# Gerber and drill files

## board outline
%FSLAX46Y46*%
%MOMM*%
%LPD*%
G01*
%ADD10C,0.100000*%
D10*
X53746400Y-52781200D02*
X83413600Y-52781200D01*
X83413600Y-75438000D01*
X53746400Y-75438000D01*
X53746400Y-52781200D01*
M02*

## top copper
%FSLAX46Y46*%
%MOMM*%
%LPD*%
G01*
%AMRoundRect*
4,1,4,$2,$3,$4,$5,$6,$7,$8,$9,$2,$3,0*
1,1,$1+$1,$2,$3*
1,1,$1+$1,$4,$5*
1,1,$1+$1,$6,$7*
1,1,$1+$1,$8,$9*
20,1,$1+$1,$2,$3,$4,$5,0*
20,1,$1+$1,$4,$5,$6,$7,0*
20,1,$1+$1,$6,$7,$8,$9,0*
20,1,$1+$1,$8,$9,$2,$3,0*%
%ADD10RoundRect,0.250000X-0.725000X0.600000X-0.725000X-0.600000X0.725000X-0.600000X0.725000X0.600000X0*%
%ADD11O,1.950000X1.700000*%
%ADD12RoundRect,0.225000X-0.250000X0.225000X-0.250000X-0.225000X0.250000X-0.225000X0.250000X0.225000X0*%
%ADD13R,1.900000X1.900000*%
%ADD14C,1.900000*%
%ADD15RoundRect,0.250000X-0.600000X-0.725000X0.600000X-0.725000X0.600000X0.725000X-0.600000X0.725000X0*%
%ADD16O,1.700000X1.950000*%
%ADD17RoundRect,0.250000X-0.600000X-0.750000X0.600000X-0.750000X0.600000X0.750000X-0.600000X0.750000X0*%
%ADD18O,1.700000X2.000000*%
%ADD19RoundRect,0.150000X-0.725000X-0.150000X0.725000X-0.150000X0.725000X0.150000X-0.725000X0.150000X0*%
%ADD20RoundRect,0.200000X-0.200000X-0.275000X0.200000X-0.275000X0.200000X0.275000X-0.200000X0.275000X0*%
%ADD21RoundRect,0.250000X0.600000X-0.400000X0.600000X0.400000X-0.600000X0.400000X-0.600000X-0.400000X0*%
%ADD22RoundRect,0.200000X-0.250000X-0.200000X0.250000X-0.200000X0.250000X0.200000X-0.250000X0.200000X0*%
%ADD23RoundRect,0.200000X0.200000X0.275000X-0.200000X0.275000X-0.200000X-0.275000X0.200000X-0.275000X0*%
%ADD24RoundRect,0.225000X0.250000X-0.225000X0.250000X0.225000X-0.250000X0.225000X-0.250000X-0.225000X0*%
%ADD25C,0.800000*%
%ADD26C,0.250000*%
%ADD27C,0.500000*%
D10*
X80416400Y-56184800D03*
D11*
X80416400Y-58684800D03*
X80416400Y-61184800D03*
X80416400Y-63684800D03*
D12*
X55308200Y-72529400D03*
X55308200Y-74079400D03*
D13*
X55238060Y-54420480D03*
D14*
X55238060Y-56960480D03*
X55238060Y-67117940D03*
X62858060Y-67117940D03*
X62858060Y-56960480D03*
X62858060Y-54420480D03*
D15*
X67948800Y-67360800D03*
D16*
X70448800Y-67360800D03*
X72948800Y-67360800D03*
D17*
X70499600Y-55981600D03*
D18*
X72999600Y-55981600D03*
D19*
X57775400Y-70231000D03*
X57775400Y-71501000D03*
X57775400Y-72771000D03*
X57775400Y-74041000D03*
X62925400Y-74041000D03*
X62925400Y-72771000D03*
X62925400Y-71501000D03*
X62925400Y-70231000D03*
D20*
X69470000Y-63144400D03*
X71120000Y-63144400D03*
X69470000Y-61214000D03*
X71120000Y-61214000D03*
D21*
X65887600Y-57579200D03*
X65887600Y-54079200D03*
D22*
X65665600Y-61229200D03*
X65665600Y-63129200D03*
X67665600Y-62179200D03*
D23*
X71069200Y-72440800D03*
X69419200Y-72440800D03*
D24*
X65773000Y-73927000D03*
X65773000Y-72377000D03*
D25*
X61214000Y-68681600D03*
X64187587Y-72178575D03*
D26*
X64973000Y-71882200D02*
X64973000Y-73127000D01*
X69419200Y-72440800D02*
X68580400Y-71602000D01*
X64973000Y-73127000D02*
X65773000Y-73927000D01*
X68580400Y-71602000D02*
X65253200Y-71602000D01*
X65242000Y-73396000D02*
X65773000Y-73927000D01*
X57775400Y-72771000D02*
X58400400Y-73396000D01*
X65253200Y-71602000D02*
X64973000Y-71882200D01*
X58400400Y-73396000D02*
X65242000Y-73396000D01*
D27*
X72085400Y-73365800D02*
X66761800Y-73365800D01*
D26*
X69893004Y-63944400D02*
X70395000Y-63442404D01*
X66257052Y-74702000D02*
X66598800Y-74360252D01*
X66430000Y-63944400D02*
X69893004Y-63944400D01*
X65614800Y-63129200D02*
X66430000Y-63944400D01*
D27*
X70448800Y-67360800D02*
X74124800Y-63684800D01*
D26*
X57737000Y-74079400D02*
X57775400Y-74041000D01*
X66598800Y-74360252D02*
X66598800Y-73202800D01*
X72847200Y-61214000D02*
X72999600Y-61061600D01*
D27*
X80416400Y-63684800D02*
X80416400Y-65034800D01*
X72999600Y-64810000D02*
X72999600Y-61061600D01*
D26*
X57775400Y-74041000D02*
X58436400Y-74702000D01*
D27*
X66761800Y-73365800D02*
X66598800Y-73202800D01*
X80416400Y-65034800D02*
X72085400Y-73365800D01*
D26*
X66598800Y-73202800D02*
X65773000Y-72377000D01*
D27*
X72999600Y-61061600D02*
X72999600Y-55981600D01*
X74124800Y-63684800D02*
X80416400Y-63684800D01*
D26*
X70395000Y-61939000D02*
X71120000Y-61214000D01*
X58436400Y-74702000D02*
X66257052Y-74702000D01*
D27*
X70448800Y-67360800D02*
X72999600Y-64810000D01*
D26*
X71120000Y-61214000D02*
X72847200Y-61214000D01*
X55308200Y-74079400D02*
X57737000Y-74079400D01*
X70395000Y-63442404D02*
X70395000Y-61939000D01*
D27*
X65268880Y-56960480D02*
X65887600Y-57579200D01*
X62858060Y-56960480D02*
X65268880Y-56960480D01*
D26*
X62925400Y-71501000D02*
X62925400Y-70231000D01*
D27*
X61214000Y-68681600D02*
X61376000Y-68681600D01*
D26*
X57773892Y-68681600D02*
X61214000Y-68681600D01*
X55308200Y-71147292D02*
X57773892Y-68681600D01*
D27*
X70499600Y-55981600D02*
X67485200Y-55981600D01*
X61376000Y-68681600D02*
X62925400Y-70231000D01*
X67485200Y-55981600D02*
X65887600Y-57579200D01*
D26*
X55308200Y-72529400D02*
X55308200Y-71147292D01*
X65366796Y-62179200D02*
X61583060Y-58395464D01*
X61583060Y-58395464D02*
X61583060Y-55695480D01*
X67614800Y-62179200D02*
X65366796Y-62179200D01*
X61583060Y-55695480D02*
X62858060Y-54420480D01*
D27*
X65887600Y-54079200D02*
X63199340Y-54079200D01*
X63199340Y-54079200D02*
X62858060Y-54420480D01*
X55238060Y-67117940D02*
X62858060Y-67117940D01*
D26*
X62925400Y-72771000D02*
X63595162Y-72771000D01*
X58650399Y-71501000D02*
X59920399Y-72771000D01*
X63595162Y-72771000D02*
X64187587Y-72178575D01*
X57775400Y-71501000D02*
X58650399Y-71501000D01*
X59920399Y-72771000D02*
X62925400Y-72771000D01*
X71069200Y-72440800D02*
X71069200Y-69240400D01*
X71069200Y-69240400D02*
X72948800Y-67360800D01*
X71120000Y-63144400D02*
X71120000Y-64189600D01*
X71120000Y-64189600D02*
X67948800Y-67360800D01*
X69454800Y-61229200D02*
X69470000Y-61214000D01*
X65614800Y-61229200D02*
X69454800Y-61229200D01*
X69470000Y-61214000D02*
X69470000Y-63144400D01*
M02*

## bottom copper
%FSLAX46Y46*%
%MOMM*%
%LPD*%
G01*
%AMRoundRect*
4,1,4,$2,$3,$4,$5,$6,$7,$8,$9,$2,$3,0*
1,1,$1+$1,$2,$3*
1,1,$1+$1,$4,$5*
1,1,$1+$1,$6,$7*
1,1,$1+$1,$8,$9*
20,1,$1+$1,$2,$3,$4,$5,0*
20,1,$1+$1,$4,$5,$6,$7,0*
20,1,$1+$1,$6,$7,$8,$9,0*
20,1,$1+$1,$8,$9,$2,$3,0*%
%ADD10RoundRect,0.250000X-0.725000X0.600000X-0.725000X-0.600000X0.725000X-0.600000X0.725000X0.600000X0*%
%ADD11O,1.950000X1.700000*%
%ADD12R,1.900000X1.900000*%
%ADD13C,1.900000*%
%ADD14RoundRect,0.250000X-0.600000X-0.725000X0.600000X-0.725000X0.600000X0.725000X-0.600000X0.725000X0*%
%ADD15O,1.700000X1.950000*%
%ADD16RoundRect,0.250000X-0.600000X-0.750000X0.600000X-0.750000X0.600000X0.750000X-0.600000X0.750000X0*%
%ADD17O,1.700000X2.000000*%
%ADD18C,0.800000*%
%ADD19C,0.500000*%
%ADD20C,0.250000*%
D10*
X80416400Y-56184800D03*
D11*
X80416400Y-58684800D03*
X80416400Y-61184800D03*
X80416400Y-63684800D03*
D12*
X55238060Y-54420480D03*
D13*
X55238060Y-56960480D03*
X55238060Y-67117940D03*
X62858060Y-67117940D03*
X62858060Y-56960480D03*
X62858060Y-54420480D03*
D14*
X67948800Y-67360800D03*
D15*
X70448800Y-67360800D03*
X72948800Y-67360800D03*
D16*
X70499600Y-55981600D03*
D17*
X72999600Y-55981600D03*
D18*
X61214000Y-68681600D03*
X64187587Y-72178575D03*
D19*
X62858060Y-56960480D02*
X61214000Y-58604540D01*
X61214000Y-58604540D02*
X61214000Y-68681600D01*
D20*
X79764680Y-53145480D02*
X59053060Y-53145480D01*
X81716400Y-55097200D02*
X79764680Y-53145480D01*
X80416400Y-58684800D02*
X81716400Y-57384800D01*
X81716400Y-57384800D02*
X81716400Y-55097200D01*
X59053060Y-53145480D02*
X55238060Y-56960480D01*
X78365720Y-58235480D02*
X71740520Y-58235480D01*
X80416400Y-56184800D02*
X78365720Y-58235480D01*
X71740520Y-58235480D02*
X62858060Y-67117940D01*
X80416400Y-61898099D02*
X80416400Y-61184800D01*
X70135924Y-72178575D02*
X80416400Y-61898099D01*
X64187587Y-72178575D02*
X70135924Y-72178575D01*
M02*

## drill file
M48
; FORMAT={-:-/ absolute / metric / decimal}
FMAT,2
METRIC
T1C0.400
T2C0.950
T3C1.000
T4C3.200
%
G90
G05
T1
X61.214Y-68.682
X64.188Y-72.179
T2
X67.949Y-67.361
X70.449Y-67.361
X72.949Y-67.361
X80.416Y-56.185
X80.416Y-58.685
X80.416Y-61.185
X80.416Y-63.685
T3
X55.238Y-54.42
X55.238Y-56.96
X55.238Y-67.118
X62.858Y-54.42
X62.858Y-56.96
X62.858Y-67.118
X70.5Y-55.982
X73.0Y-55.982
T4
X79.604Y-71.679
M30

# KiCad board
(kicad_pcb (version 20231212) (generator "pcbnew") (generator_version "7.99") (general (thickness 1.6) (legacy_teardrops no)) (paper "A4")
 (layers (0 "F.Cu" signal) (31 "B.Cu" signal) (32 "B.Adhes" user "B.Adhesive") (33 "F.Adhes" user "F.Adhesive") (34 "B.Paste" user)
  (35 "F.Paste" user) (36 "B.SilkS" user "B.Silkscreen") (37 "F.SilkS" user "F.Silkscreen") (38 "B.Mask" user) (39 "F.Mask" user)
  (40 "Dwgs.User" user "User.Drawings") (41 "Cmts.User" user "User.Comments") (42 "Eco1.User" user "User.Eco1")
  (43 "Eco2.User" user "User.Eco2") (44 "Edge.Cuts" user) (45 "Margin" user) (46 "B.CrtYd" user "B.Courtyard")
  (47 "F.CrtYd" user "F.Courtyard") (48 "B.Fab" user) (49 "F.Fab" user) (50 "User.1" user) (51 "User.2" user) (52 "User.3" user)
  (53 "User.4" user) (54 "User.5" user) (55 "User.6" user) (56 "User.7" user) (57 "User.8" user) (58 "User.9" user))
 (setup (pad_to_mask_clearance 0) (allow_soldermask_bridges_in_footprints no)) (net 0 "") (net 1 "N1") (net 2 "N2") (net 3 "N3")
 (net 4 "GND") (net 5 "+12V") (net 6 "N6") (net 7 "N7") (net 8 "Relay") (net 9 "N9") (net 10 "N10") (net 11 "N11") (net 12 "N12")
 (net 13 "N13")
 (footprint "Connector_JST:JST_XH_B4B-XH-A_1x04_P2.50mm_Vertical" (layer "F.Cu") (at 80.4164 56.1848 -90)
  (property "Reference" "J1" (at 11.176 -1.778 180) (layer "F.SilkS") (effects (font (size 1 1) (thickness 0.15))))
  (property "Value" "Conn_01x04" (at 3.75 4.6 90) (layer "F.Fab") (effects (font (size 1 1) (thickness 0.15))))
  (pad "1" thru_hole roundrect (at 0 0 270) (size 1.7 1.95) (drill 0.95) (layers "*.Cu" "*.Mask") (remove_unused_layers no)
   (roundrect_rratio 0.1470588235) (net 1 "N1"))
  (pad "2" thru_hole oval (at 2.5 0 270) (size 1.7 1.95) (drill 0.95) (layers "*.Cu" "*.Mask") (remove_unused_layers no) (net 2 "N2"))
  (pad "3" thru_hole oval (at 5 0 270) (size 1.7 1.95) (drill 0.95) (layers "*.Cu" "*.Mask") (remove_unused_layers no) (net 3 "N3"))
  (pad "4" thru_hole oval (at 7.5 0 270) (size 1.7 1.95) (drill 0.95) (layers "*.Cu" "*.Mask") (remove_unused_layers no) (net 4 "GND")))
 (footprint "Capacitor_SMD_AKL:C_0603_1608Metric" (layer "F.Cu") (at 55.3082 73.3044 -90)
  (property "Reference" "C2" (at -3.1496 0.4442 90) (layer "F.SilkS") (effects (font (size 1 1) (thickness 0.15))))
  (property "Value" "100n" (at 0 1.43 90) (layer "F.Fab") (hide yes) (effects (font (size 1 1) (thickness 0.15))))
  (pad "1" smd roundrect (at -0.775 0 270) (size 0.9 0.95) (layers "F.Cu" "F.Paste" "F.Mask") (roundrect_rratio 0.25) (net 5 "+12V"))
  (pad "2" smd roundrect (at 0.775 0 270) (size 0.9 0.95) (layers "F.Cu" "F.Paste" "F.Mask") (roundrect_rratio 0.25) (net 4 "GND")))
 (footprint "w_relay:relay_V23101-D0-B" (layer "F.Cu") (at 59.04806 60.92034)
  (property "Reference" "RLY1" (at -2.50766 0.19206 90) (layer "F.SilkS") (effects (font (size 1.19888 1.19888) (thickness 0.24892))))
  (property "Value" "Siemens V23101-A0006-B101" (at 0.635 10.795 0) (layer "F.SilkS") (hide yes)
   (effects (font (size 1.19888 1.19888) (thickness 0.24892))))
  (pad "1" thru_hole rect (at -3.81 -6.49986) (size 1.9 1.9) (drill 1) (layers "*.Cu" "*.Mask" "F.SilkS") (remove_unused_layers no)
   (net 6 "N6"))
  (pad "2" thru_hole circle (at -3.81 -3.95986) (size 1.9 1.9) (drill 1) (layers "*.Cu" "*.Mask" "F.SilkS") (remove_unused_layers no)
   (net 2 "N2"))
  (pad "6" thru_hole circle (at -3.81 6.1976) (size 1.9 1.9) (drill 1) (layers "*.Cu" "*.Mask" "F.SilkS") (remove_unused_layers no)
   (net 1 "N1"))
  (pad "7" thru_hole circle (at 3.81 6.1976) (size 1.9 1.9) (drill 1) (layers "*.Cu" "*.Mask" "F.SilkS") (remove_unused_layers no)
   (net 1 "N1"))
  (pad "11" thru_hole circle (at 3.81 -3.95986) (size 1.9 1.9) (drill 1) (layers "*.Cu" "*.Mask" "F.SilkS") (remove_unused_layers no)
   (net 5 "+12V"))
  (pad "12" thru_hole circle (at 3.81 -6.49986) (size 1.9 1.9) (drill 1) (layers "*.Cu" "*.Mask" "F.SilkS") (remove_unused_layers no)
   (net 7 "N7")))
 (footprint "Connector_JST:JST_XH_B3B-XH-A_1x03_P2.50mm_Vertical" (layer "F.Cu") (at 67.9488 67.3608)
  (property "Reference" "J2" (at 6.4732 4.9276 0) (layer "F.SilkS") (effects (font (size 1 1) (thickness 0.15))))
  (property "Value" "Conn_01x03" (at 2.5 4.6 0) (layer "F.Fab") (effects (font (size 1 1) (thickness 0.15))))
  (pad "1" thru_hole roundrect (at 0 0) (size 1.7 1.95) (drill 0.95) (layers "*.Cu" "*.Mask") (remove_unused_layers no)
   (roundrect_rratio 0.1470588235) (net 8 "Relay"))
  (pad "2" thru_hole oval (at 2.5 0) (size 1.7 1.95) (drill 0.95) (layers "*.Cu" "*.Mask") (remove_unused_layers no) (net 4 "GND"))
  (pad "3" thru_hole oval (at 5 0) (size 1.7 1.95) (drill 0.95) (layers "*.Cu" "*.Mask") (remove_unused_layers no) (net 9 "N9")))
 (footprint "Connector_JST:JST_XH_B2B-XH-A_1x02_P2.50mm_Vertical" (layer "F.Cu") (at 70.4996 55.9816)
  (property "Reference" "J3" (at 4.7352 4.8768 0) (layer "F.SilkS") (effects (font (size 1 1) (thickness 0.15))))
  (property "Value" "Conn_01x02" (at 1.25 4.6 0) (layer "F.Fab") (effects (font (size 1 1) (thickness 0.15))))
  (pad "1" thru_hole roundrect (at 0 0) (size 1.7 2) (drill 1) (layers "*.Cu" "*.Mask") (remove_unused_layers no)
   (roundrect_rratio 0.1470588235) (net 5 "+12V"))
  (pad "2" thru_hole oval (at 2.5 0) (size 1.7 2) (drill 1) (layers "*.Cu" "*.Mask") (remove_unused_layers no) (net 4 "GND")))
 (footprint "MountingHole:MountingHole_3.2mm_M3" (layer "F.Cu") (at 79.6036 71.6788)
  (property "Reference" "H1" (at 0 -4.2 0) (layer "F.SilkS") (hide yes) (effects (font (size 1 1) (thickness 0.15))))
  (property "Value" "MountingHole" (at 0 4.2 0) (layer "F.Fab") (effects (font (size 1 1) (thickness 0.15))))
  (pad "" np_thru_hole circle (at 0 0) (size 3.2 3.2) (drill 3.2) (layers "*.Cu" "*.Mask")))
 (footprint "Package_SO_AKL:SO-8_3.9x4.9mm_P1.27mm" (layer "F.Cu") (at 60.3504 72.136)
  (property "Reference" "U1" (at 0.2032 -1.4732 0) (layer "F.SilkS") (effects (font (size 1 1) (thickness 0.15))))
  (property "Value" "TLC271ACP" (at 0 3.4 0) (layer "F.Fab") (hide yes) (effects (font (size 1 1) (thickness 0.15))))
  (pad "1" smd roundrect (at -2.575 -1.905) (size 1.75 0.6) (layers "F.Cu" "F.Paste" "F.Mask") (roundrect_rratio 0.25) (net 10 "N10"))
  (pad "2" smd roundrect (at -2.575 -0.635) (size 1.75 0.6) (layers "F.Cu" "F.Paste" "F.Mask") (roundrect_rratio 0.25) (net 3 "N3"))
  (pad "3" smd roundrect (at -2.575 0.635) (size 1.75 0.6) (layers "F.Cu" "F.Paste" "F.Mask") (roundrect_rratio 0.25) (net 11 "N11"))
  (pad "4" smd roundrect (at -2.575 1.905) (size 1.75 0.6) (layers "F.Cu" "F.Paste" "F.Mask") (roundrect_rratio 0.25) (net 4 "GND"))
  (pad "5" smd roundrect (at 2.575 1.905) (size 1.75 0.6) (layers "F.Cu" "F.Paste" "F.Mask") (roundrect_rratio 0.25) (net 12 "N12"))
  (pad "6" smd roundrect (at 2.575 0.635) (size 1.75 0.6) (layers "F.Cu" "F.Paste" "F.Mask") (roundrect_rratio 0.25) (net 3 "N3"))
  (pad "7" smd roundrect (at 2.575 -0.635) (size 1.75 0.6) (layers "F.Cu" "F.Paste" "F.Mask") (roundrect_rratio 0.25) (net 5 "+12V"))
  (pad "8" smd roundrect (at 2.575 -1.905) (size 1.75 0.6) (layers "F.Cu" "F.Paste" "F.Mask") (roundrect_rratio 0.25) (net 5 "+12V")))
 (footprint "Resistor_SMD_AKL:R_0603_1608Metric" (layer "F.Cu") (at 70.295 63.1444)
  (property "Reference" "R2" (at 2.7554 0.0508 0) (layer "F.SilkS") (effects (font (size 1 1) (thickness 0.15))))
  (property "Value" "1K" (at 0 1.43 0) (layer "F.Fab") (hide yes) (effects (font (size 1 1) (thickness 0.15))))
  (pad "1" smd roundrect (at -0.825 0) (size 0.8 0.95) (layers "F.Cu" "F.Paste" "F.Mask") (roundrect_rratio 0.25) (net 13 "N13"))
  (pad "2" smd roundrect (at 0.825 0) (size 0.8 0.95) (layers "F.Cu" "F.Paste" "F.Mask") (roundrect_rratio 0.25) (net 8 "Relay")))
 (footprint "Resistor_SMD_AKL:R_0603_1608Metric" (layer "F.Cu") (at 70.295 61.214)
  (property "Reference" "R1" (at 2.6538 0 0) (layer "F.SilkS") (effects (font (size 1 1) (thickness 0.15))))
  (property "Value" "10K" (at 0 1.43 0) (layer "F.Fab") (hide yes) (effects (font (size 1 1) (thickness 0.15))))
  (pad "1" smd roundrect (at -0.825 0) (size 0.8 0.95) (layers "F.Cu" "F.Paste" "F.Mask") (roundrect_rratio 0.25) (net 13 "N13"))
  (pad "2" smd roundrect (at 0.825 0) (size 0.8 0.95) (layers "F.Cu" "F.Paste" "F.Mask") (roundrect_rratio 0.25) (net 4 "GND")))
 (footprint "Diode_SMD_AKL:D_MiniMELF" (layer "F.Cu") (at 65.8876 55.8292 90)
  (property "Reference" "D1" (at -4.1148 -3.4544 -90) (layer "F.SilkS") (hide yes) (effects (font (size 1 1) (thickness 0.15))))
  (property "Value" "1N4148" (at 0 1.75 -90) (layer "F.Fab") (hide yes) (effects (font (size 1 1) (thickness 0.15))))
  (pad "1" smd roundrect (at -1.75 0 90) (size 1.3 1.7) (layers "F.Cu" "F.Paste" "F.Mask") (roundrect_rratio 0.1923076923) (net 5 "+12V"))
  (pad "2" smd roundrect (at 1.75 0 90) (size 1.3 1.7) (layers "F.Cu" "F.Paste" "F.Mask") (roundrect_rratio 0.1923076923) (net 7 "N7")))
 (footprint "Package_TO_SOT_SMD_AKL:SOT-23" (layer "F.Cu") (at 66.6656 62.1792)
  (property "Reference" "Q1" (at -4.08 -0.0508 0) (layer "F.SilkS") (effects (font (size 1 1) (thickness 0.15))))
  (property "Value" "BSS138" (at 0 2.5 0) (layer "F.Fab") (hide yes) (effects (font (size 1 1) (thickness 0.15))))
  (pad "1" smd roundrect (at -1 -0.95) (size 0.9 0.8) (layers "F.Cu" "F.Paste" "F.Mask") (roundrect_rratio 0.25) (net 13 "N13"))
  (pad "2" smd roundrect (at -1 0.95) (size 0.9 0.8) (layers "F.Cu" "F.Paste" "F.Mask") (roundrect_rratio 0.25) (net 4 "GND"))
  (pad "3" smd roundrect (at 1 0) (size 0.9 0.8) (layers "F.Cu" "F.Paste" "F.Mask") (roundrect_rratio 0.25) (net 7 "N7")))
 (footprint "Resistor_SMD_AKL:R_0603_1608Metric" (layer "F.Cu") (at 70.2442 72.4408 180)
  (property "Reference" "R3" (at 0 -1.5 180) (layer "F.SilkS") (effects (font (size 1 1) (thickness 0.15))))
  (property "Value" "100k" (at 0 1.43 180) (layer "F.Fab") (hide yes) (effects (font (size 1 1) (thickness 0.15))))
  (pad "1" smd roundrect (at -0.825 0 180) (size 0.8 0.95) (layers "F.Cu" "F.Paste" "F.Mask") (roundrect_rratio 0.25) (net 9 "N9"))
  (pad "2" smd roundrect (at 0.825 0 180) (size 0.8 0.95) (layers "F.Cu" "F.Paste" "F.Mask") (roundrect_rratio 0.25) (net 11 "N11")))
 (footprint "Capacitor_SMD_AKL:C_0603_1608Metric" (layer "F.Cu") (at 65.773 73.152 90)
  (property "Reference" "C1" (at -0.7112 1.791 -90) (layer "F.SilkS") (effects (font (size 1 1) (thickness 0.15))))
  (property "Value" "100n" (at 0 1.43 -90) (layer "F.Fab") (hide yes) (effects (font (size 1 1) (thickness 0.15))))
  (pad "1" smd roundrect (at -0.775 0 90) (size 0.9 0.95) (layers "F.Cu" "F.Paste" "F.Mask") (roundrect_rratio 0.25) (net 11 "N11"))
  (pad "2" smd roundrect (at 0.775 0 90) (size 0.9 0.95) (layers "F.Cu" "F.Paste" "F.Mask") (roundrect_rratio 0.25) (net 4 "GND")))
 (gr_rect (start 53.7464 52.7812) (end 83.4136 75.438) (stroke (width 0.1) (type default)) (fill none) (layer "Edge.Cuts"))
 (segment (start 64.973 71.8822) (end 64.973 73.127) (width 0.25) (layer "F.Cu") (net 11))
 (segment (start 69.4192 72.4408) (end 68.5804 71.602) (width 0.25) (layer "F.Cu") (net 11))
 (segment (start 64.973 73.127) (end 65.773 73.927) (width 0.25) (layer "F.Cu") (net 11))
 (segment (start 68.5804 71.602) (end 65.2532 71.602) (width 0.25) (layer "F.Cu") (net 11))
 (segment (start 65.242 73.396) (end 65.773 73.927) (width 0.25) (layer "F.Cu") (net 11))
 (segment (start 57.7754 72.771) (end 58.4004 73.396) (width 0.25) (layer "F.Cu") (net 11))
 (segment (start 65.2532 71.602) (end 64.973 71.8822) (width 0.25) (layer "F.Cu") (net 11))
 (segment (start 58.4004 73.396) (end 65.242 73.396) (width 0.25) (layer "F.Cu") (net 11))
 (segment (start 72.0854 73.3658) (end 66.7618 73.3658) (width 0.5) (layer "F.Cu") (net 4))
 (segment (start 69.893004 63.9444) (end 70.395 63.442404) (width 0.25) (layer "F.Cu") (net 4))
 (segment (start 66.257052 74.702) (end 66.5988 74.360252) (width 0.25) (layer "F.Cu") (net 4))
 (segment (start 66.43 63.9444) (end 69.893004 63.9444) (width 0.25) (layer "F.Cu") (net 4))
 (segment (start 65.6148 63.1292) (end 66.43 63.9444) (width 0.25) (layer "F.Cu") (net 4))
 (segment (start 70.4488 67.3608) (end 74.1248 63.6848) (width 0.5) (layer "F.Cu") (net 4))
 (segment (start 57.737 74.0794) (end 57.7754 74.041) (width 0.25) (layer "F.Cu") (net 4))
 (segment (start 66.5988 74.360252) (end 66.5988 73.2028) (width 0.25) (layer "F.Cu") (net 4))
 (segment (start 72.8472 61.214) (end 72.9996 61.0616) (width 0.25) (layer "F.Cu") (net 4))
 (segment (start 80.4164 63.6848) (end 80.4164 65.0348) (width 0.5) (layer "F.Cu") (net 4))
 (segment (start 72.9996 64.81) (end 72.9996 61.0616) (width 0.5) (layer "F.Cu") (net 4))
 (segment (start 57.7754 74.041) (end 58.4364 74.702) (width 0.25) (layer "F.Cu") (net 4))
 (segment (start 66.7618 73.3658) (end 66.5988 73.2028) (width 0.5) (layer "F.Cu") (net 4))
 (segment (start 80.4164 65.0348) (end 72.0854 73.3658) (width 0.5) (layer "F.Cu") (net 4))
 (segment (start 66.5988 73.2028) (end 65.773 72.377) (width 0.25) (layer "F.Cu") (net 4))
 (segment (start 72.9996 61.0616) (end 72.9996 55.9816) (width 0.5) (layer "F.Cu") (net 4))
 (segment (start 74.1248 63.6848) (end 80.4164 63.6848) (width 0.5) (layer "F.Cu") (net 4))
 (segment (start 70.395 61.939) (end 71.12 61.214) (width 0.25) (layer "F.Cu") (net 4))
 (segment (start 58.4364 74.702) (end 66.257052 74.702) (width 0.25) (layer "F.Cu") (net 4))
 (segment (start 70.4488 67.3608) (end 72.9996 64.81) (width 0.5) (layer "F.Cu") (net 4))
 (segment (start 71.12 61.214) (end 72.8472 61.214) (width 0.25) (layer "F.Cu") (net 4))
 (segment (start 55.3082 74.0794) (end 57.737 74.0794) (width 0.25) (layer "F.Cu") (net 4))
 (segment (start 70.395 63.442404) (end 70.395 61.939) (width 0.25) (layer "F.Cu") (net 4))
 (segment (start 65.26888 56.96048) (end 65.8876 57.5792) (width 0.5) (layer "F.Cu") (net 5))
 (segment (start 62.85806 56.96048) (end 65.26888 56.96048) (width 0.5) (layer "F.Cu") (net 5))
 (segment (start 62.9254 71.501) (end 62.9254 70.231) (width 0.25) (layer "F.Cu") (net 5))
 (segment (start 61.214 68.6816) (end 61.376 68.6816) (width 0.5) (layer "F.Cu") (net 5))
 (segment (start 57.773892 68.6816) (end 61.214 68.6816) (width 0.25) (layer "F.Cu") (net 5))
 (segment (start 55.3082 71.147292) (end 57.773892 68.6816) (width 0.25) (layer "F.Cu") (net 5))
 (segment (start 70.4996 55.9816) (end 67.4852 55.9816) (width 0.5) (layer "F.Cu") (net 5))
 (segment (start 61.376 68.6816) (end 62.9254 70.231) (width 0.5) (layer "F.Cu") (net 5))
 (segment (start 67.4852 55.9816) (end 65.8876 57.5792) (width 0.5) (layer "F.Cu") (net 5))
 (segment (start 55.3082 72.5294) (end 55.3082 71.147292) (width 0.25) (layer "F.Cu") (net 5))
 (via (at 61.214 68.6816) (size 0.8) (drill 0.4) (layers "F.Cu" "B.Cu") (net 5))
 (segment (start 62.85806 56.96048) (end 61.214 58.60454) (width 0.5) (layer "B.Cu") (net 5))
 (segment (start 61.214 58.60454) (end 61.214 68.6816) (width 0.5) (layer "B.Cu") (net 5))
 (segment (start 65.366796 62.1792) (end 61.58306 58.395464) (width 0.25) (layer "F.Cu") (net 7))
 (segment (start 61.58306 58.395464) (end 61.58306 55.69548) (width 0.25) (layer "F.Cu") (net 7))
 (segment (start 67.6148 62.1792) (end 65.366796 62.1792) (width 0.25) (layer "F.Cu") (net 7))
 (segment (start 61.58306 55.69548) (end 62.85806 54.42048) (width 0.25) (layer "F.Cu") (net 7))
 (segment (start 65.8876 54.0792) (end 63.19934 54.0792) (width 0.5) (layer "F.Cu") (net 7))
 (segment (start 63.19934 54.0792) (end 62.85806 54.42048) (width 0.5) (layer "F.Cu") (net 7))
 (segment (start 79.76468 53.14548) (end 59.05306 53.14548) (width 0.25) (layer "B.Cu") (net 2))
 (segment (start 81.7164 55.0972) (end 79.76468 53.14548) (width 0.25) (layer "B.Cu") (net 2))
 (segment (start 80.4164 58.6848) (end 81.7164 57.3848) (width 0.25) (layer "B.Cu") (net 2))
 (segment (start 81.7164 57.3848) (end 81.7164 55.0972) (width 0.25) (layer "B.Cu") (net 2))
 (segment (start 59.05306 53.14548) (end 55.23806 56.96048) (width 0.25) (layer "B.Cu") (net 2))
 (segment (start 55.23806 67.11794) (end 62.85806 67.11794) (width 0.5) (layer "F.Cu") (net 1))
 (segment (start 78.36572 58.23548) (end 71.74052 58.23548) (width 0.25) (layer "B.Cu") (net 1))
 (segment (start 80.4164 56.1848) (end 78.36572 58.23548) (width 0.25) (layer "B.Cu") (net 1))
 (segment (start 71.74052 58.23548) (end 62.85806 67.11794) (width 0.25) (layer "B.Cu") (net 1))
 (segment (start 62.9254 72.771) (end 63.595162 72.771) (width 0.25) (layer "F.Cu") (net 3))
 (segment (start 58.650399 71.501) (end 59.920399 72.771) (width 0.25) (layer "F.Cu") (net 3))
 (segment (start 63.595162 72.771) (end 64.187587 72.178575) (width 0.25) (layer "F.Cu") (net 3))
 (segment (start 57.7754 71.501) (end 58.650399 71.501) (width 0.25) (layer "F.Cu") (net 3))
 (segment (start 59.920399 72.771) (end 62.9254 72.771) (width 0.25) (layer "F.Cu") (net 3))
 (via (at 64.187587 72.178575) (size 0.8) (drill 0.4) (layers "F.Cu" "B.Cu") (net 3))
 (segment (start 80.4164 61.898099) (end 80.4164 61.1848) (width 0.25) (layer "B.Cu") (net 3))
 (segment (start 70.135924 72.178575) (end 80.4164 61.898099) (width 0.25) (layer "B.Cu") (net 3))
 (segment (start 64.187587 72.178575) (end 70.135924 72.178575) (width 0.25) (layer "B.Cu") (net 3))
 (segment (start 71.0692 72.4408) (end 71.0692 69.2404) (width 0.25) (layer "F.Cu") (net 9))
 (segment (start 71.0692 69.2404) (end 72.9488 67.3608) (width 0.25) (layer "F.Cu") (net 9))
 (segment (start 71.12 63.1444) (end 71.12 64.1896) (width 0.25) (layer "F.Cu") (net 8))
 (segment (start 71.12 64.1896) (end 67.9488 67.3608) (width 0.25) (layer "F.Cu") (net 8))
 (segment (start 69.4548 61.2292) (end 69.47 61.214) (width 0.25) (layer "F.Cu") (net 13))
 (segment (start 65.6148 61.2292) (end 69.4548 61.2292) (width 0.25) (layer "F.Cu") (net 13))
 (segment (start 69.47 61.214) (end 69.47 63.1444) (width 0.25) (layer "F.Cu") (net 13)))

